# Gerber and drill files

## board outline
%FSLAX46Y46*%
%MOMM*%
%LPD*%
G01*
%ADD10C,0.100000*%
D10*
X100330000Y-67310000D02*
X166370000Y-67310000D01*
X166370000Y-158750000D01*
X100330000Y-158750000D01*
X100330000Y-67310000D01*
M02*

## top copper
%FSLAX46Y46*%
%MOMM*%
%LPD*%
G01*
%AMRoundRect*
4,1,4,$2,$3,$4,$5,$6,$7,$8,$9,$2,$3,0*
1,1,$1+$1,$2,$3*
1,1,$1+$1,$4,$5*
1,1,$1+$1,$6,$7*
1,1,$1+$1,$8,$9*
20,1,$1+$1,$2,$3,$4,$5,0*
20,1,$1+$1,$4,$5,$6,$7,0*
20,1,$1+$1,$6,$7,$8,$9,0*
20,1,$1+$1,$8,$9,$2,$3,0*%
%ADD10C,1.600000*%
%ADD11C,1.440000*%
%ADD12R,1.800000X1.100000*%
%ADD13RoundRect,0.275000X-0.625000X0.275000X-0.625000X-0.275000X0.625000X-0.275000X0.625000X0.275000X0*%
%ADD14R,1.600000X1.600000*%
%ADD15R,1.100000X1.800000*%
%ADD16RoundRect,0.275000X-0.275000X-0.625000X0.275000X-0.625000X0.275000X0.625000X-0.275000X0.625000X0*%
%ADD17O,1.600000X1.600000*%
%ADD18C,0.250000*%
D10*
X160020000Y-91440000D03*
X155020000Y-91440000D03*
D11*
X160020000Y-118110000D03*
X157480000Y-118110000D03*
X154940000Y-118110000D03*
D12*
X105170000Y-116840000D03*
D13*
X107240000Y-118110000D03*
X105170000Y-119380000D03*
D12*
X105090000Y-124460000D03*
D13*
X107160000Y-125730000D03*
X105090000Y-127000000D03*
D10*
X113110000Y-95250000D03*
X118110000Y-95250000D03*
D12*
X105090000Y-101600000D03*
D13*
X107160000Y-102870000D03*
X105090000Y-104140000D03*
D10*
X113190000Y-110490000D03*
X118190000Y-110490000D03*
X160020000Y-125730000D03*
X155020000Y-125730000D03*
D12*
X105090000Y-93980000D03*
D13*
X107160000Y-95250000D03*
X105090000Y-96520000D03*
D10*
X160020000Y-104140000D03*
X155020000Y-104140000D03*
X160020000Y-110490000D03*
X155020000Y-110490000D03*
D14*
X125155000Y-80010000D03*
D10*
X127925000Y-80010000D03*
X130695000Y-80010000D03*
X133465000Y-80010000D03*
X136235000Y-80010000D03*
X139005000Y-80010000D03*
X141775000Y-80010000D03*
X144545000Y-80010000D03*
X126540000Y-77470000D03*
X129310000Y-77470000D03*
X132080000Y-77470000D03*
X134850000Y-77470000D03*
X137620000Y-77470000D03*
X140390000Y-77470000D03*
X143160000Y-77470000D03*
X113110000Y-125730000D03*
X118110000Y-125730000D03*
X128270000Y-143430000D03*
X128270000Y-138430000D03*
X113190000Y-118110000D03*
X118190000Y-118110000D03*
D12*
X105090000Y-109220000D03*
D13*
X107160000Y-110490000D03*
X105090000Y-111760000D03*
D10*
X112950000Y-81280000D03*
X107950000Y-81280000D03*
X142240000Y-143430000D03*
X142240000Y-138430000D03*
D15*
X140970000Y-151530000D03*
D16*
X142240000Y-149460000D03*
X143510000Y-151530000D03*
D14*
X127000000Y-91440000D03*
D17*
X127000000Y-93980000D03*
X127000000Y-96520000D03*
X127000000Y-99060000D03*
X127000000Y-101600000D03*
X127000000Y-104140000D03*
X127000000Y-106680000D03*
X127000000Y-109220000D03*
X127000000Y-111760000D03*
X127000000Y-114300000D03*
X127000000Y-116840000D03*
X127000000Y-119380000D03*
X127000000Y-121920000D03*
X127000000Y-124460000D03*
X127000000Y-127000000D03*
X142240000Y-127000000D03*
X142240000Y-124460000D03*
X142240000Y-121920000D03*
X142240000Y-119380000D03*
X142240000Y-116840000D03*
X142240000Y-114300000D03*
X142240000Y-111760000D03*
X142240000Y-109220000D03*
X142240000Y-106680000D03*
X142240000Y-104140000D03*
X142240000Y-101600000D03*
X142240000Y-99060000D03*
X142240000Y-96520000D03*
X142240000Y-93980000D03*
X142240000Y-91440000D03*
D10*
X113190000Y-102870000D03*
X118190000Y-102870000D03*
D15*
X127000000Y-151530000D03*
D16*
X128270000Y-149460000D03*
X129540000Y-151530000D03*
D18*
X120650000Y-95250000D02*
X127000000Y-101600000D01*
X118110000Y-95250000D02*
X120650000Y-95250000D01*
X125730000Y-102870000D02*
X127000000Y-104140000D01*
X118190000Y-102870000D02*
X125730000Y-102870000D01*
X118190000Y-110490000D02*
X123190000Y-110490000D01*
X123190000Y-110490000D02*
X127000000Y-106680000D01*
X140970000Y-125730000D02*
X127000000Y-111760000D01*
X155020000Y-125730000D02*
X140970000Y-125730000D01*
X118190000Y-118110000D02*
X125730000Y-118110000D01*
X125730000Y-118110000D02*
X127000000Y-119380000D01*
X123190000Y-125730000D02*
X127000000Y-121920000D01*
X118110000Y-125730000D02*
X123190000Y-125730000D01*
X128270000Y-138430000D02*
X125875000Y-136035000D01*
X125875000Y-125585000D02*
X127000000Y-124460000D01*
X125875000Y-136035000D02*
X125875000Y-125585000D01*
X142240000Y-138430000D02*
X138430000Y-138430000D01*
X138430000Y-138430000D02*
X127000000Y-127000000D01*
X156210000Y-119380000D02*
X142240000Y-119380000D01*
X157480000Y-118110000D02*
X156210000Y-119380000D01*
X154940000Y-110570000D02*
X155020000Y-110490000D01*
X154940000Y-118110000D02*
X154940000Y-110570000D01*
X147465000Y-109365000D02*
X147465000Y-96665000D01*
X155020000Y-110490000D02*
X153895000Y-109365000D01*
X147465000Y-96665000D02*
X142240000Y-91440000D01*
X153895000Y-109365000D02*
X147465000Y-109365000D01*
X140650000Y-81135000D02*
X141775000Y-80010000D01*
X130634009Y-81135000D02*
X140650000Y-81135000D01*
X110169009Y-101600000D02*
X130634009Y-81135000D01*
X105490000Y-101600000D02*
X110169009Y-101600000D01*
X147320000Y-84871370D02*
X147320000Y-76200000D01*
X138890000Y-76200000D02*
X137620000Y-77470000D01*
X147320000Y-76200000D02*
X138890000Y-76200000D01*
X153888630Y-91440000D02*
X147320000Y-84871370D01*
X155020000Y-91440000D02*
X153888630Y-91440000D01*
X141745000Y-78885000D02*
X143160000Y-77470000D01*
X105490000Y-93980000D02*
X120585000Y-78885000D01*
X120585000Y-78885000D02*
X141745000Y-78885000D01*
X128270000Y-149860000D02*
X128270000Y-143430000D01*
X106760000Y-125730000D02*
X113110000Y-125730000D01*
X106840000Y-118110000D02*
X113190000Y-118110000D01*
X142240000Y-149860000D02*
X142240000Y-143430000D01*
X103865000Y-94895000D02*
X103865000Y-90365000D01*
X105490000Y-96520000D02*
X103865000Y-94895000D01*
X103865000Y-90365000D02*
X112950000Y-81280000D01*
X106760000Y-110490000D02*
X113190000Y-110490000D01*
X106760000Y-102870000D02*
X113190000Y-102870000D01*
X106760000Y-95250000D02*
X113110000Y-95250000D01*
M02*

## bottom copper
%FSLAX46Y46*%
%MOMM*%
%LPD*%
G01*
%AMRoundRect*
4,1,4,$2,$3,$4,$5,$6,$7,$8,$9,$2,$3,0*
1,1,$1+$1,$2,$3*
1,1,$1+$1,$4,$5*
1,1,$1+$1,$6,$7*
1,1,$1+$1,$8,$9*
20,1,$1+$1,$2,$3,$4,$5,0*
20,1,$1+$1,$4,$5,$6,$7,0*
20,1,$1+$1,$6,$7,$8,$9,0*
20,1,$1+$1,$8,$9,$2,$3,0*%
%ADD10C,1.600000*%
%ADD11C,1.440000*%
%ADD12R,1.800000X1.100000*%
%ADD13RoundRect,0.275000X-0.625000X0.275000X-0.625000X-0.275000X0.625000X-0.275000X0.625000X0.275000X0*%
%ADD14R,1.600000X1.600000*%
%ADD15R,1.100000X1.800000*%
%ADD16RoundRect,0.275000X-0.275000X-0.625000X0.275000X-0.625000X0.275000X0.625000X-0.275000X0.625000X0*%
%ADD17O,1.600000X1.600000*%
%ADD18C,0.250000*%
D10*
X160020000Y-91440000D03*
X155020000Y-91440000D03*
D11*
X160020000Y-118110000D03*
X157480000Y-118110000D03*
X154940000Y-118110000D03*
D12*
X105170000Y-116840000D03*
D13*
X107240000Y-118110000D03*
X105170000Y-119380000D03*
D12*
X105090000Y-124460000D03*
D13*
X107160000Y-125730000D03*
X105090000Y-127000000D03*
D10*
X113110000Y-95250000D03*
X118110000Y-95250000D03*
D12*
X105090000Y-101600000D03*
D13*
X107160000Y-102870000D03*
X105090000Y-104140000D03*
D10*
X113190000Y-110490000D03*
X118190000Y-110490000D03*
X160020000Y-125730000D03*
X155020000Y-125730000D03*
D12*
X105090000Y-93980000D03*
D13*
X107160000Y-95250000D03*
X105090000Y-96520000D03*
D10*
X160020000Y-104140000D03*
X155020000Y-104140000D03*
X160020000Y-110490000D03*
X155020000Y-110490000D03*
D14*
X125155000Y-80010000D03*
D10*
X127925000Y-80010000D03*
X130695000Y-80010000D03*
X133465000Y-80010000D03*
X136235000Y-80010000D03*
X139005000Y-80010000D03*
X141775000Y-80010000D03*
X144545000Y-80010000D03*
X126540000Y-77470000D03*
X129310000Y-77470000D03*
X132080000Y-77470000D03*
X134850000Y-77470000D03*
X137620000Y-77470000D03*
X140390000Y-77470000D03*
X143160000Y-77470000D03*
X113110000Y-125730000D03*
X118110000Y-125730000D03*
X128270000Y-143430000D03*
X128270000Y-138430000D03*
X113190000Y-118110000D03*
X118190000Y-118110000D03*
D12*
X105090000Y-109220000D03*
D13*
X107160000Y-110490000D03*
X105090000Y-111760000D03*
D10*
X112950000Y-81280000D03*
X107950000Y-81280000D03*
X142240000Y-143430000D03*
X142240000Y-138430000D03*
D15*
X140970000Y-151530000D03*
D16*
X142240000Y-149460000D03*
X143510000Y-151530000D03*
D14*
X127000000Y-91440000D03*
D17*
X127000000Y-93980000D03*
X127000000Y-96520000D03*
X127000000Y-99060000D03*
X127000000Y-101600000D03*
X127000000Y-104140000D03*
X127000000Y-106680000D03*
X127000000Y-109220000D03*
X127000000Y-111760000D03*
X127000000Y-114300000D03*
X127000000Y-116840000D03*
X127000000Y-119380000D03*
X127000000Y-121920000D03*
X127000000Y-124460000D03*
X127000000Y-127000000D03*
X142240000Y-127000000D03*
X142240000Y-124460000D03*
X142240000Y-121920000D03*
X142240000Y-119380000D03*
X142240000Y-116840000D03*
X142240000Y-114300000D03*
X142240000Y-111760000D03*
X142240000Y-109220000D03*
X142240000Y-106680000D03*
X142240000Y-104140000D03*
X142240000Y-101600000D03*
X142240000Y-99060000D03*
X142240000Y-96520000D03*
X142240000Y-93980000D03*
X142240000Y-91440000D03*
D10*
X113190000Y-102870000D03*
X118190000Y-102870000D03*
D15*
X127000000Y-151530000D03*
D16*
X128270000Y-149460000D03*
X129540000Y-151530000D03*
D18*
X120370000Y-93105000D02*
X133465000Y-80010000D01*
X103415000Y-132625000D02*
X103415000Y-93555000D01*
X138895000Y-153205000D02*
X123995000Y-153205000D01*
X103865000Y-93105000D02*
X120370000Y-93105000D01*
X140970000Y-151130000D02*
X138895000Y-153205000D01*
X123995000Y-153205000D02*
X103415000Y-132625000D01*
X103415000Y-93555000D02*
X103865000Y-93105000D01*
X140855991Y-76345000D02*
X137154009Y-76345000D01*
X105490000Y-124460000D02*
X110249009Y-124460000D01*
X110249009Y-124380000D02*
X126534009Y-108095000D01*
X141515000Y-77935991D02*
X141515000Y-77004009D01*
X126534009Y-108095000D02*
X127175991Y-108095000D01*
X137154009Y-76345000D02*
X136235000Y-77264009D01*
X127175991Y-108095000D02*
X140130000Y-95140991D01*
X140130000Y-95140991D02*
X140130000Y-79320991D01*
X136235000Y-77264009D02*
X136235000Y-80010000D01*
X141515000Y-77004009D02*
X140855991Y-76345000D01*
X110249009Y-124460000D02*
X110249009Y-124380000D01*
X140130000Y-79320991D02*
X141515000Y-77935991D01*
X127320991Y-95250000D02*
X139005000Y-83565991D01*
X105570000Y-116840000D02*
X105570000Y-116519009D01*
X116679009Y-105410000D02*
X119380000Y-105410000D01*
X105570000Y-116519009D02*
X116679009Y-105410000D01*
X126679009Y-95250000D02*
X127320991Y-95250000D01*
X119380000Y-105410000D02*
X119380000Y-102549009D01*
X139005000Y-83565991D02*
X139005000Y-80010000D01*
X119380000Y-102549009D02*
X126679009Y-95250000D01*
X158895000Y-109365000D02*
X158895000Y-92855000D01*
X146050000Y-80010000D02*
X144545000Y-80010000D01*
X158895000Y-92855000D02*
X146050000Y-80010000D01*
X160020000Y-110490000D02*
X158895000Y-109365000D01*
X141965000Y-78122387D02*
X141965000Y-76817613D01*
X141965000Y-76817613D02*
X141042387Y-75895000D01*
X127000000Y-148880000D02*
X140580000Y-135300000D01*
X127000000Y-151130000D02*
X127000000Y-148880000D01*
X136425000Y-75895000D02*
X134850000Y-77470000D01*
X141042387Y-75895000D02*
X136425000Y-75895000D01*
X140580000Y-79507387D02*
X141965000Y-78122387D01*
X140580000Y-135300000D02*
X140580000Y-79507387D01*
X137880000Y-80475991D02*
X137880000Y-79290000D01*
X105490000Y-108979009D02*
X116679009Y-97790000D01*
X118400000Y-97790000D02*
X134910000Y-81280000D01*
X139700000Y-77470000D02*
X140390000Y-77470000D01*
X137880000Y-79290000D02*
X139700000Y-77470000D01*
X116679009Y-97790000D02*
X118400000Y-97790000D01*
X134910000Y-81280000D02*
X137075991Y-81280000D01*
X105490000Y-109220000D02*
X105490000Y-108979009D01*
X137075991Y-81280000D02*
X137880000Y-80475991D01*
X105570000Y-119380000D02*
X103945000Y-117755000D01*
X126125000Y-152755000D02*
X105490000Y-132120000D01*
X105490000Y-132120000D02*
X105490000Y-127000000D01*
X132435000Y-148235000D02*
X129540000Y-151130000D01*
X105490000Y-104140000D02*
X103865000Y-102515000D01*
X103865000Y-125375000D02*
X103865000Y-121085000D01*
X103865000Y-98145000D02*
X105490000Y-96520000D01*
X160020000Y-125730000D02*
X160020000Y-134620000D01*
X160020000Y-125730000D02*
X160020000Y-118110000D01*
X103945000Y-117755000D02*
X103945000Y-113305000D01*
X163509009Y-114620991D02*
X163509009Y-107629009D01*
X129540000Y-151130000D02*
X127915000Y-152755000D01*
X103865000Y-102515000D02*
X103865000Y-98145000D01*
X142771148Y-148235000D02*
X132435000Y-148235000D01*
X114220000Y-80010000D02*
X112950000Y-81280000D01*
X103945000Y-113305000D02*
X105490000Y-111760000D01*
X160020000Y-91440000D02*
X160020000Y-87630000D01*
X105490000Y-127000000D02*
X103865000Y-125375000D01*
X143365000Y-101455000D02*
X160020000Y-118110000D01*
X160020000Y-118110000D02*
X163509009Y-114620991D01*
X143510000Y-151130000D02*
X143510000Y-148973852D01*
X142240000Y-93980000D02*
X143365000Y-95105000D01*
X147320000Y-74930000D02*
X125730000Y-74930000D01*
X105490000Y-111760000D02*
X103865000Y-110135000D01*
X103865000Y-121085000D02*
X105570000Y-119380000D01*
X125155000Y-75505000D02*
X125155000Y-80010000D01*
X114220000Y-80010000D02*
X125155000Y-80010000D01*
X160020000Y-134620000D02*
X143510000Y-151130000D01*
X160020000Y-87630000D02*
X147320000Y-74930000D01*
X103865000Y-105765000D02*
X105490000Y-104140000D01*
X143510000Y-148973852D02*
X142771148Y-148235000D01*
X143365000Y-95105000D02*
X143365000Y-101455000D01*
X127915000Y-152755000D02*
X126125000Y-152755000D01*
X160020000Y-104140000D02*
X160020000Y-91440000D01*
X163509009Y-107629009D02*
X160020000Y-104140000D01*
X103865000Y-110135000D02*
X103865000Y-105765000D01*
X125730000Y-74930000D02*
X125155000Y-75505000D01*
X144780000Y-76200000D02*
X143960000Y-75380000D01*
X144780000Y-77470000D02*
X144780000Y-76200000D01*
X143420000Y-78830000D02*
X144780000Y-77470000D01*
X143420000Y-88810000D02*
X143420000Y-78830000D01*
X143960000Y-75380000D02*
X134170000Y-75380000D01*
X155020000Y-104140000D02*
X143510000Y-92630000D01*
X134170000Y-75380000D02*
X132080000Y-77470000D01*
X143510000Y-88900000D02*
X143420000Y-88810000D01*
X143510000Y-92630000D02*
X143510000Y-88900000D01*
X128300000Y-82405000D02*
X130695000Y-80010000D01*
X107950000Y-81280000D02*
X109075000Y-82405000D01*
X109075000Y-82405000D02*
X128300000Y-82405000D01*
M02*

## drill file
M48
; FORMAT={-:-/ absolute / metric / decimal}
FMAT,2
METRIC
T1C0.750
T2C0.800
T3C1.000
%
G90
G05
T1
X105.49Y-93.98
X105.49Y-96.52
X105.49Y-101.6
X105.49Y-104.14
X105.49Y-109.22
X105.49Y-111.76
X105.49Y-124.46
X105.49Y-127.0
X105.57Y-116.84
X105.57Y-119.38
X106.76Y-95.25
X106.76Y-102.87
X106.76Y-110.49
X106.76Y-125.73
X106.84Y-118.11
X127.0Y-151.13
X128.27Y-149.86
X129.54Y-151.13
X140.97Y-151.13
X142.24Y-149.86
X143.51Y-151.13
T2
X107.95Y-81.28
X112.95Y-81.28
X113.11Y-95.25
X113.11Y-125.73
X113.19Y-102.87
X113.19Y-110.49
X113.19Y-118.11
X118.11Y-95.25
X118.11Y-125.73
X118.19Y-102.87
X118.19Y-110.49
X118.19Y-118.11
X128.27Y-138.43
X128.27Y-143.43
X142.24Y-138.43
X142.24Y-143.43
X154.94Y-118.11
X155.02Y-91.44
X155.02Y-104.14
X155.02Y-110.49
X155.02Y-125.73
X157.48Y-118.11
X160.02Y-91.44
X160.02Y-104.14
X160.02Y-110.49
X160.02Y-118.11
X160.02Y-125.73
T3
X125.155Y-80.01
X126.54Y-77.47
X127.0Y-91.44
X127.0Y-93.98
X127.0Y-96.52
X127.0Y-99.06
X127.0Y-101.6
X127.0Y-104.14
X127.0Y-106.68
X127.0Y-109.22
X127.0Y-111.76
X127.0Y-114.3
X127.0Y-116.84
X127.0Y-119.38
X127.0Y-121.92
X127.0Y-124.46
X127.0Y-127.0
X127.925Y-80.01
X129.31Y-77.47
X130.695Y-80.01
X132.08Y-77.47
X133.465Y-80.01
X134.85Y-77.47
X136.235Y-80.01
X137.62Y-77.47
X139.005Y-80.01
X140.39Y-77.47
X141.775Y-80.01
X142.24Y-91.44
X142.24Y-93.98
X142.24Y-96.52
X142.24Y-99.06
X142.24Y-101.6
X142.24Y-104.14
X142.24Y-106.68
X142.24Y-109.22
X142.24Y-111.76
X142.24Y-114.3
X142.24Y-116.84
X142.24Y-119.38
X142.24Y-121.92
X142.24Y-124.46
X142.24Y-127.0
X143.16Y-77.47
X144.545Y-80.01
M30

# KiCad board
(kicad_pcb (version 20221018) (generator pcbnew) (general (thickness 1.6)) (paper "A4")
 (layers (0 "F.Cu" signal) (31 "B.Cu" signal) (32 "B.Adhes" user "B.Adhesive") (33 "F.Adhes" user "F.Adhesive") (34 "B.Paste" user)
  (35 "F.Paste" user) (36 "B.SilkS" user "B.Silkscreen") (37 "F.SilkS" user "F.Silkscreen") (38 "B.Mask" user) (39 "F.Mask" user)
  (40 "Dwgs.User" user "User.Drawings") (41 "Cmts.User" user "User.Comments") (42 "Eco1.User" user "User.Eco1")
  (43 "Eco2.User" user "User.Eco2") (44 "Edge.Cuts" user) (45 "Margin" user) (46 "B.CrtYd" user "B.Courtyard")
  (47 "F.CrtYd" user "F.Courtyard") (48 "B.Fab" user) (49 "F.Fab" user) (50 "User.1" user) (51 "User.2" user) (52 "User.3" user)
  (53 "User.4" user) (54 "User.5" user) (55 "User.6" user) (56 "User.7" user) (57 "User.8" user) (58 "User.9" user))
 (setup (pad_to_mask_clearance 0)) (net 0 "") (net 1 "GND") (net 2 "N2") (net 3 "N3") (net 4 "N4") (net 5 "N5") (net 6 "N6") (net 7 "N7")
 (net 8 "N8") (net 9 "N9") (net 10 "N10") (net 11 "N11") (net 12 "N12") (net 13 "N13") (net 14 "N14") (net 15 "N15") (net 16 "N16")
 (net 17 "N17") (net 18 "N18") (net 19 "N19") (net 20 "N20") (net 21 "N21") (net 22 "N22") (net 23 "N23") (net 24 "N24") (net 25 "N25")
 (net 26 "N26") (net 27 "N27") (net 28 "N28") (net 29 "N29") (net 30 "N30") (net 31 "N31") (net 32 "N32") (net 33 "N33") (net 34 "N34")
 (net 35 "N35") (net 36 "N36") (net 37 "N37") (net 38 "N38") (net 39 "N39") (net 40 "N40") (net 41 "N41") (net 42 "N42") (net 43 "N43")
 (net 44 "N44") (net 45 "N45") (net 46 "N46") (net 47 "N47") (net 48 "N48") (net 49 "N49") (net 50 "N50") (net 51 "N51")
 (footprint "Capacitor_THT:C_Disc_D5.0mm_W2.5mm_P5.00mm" (layer "F.Cu") (at 160.02 91.44 180)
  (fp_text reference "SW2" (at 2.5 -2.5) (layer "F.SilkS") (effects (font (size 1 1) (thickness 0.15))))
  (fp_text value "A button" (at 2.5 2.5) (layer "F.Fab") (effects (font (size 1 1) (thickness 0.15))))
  (pad "1" thru_hole circle (at 0 0 180) (size 1.6 1.6) (drill 0.8) (layers "*.Cu" "*.Mask") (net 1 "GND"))
  (pad "2" thru_hole circle (at 5 0 180) (size 1.6 1.6) (drill 0.8) (layers "*.Cu" "*.Mask") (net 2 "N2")))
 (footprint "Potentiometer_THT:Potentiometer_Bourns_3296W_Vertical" (layer "F.Cu") (at 160.02 118.11)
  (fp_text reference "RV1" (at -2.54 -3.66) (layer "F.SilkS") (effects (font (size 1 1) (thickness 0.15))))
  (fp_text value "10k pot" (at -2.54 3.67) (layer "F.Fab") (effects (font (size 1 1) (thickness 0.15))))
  (pad "1" thru_hole circle (at 0 0) (size 1.44 1.44) (drill 0.8) (layers "*.Cu" "*.Mask") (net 1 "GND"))
  (pad "2" thru_hole circle (at -2.54 0) (size 1.44 1.44) (drill 0.8) (layers "*.Cu" "*.Mask") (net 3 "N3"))
  (pad "3" thru_hole circle (at -5.08 0) (size 1.44 1.44) (drill 0.8) (layers "*.Cu" "*.Mask") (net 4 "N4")))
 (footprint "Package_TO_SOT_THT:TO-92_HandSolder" (layer "F.Cu") (at 105.57 116.84 -90)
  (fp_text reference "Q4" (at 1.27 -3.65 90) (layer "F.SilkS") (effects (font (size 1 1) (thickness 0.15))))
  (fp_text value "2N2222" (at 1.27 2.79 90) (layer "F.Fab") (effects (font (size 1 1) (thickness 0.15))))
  (pad "1" thru_hole rect (at 0 0 270) (size 1.1 1.8) (drill 0.75 (offset 0 0.4)) (layers "*.Cu" "*.Mask") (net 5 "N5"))
  (pad "2" thru_hole roundrect (at 1.27 -1.27 270) (size 1.1 1.8) (drill 0.75 (offset 0 -0.4)) (layers "*.Cu" "*.Mask")
   (roundrect_rratio 0.25) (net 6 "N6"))
  (pad "3" thru_hole roundrect (at 2.54 0 270) (size 1.1 1.8) (drill 0.75 (offset 0 0.4)) (layers "*.Cu" "*.Mask") (roundrect_rratio 0.25)
   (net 1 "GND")))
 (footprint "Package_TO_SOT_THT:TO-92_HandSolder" (layer "F.Cu") (at 105.49 124.46 -90)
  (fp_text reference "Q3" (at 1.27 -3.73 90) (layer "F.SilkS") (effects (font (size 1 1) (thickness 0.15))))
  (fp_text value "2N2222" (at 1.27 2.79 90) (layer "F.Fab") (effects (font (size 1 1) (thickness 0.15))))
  (pad "1" thru_hole rect (at 0 0 270) (size 1.1 1.8) (drill 0.75 (offset 0 0.4)) (layers "*.Cu" "*.Mask") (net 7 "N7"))
  (pad "2" thru_hole roundrect (at 1.27 -1.27 270) (size 1.1 1.8) (drill 0.75 (offset 0 -0.4)) (layers "*.Cu" "*.Mask")
   (roundrect_rratio 0.25) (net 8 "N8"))
  (pad "3" thru_hole roundrect (at 2.54 0 270) (size 1.1 1.8) (drill 0.75 (offset 0 0.4)) (layers "*.Cu" "*.Mask") (roundrect_rratio 0.25)
   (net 1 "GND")))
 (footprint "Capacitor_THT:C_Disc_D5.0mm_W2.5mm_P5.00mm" (layer "F.Cu") (at 113.11 95.25)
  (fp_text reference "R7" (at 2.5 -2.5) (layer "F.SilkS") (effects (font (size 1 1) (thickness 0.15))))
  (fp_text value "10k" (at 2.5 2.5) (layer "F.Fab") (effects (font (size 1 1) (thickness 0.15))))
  (pad "1" thru_hole circle (at 0 0) (size 1.6 1.6) (drill 0.8) (layers "*.Cu" "*.Mask") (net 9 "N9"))
  (pad "2" thru_hole circle (at 5 0) (size 1.6 1.6) (drill 0.8) (layers "*.Cu" "*.Mask") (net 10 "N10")))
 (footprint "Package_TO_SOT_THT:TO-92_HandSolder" (layer "F.Cu") (at 105.49 101.6 -90)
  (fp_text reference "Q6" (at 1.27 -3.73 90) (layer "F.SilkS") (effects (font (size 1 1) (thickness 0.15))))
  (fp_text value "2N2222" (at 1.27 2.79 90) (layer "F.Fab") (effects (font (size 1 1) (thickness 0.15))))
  (pad "1" thru_hole rect (at 0 0 270) (size 1.1 1.8) (drill 0.75 (offset 0 0.4)) (layers "*.Cu" "*.Mask") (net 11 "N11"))
  (pad "2" thru_hole roundrect (at 1.27 -1.27 270) (size 1.1 1.8) (drill 0.75 (offset 0 -0.4)) (layers "*.Cu" "*.Mask")
   (roundrect_rratio 0.25) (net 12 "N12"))
  (pad "3" thru_hole roundrect (at 2.54 0 270) (size 1.1 1.8) (drill 0.75 (offset 0 0.4)) (layers "*.Cu" "*.Mask") (roundrect_rratio 0.25)
   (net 1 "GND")))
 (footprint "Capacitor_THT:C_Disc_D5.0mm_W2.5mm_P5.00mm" (layer "F.Cu") (at 113.19 110.49)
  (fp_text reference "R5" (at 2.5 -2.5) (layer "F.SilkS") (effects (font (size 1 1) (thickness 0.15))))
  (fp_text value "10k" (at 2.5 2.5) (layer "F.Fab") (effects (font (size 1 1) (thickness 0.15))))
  (pad "1" thru_hole circle (at 0 0) (size 1.6 1.6) (drill 0.8) (layers "*.Cu" "*.Mask") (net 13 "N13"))
  (pad "2" thru_hole circle (at 5 0) (size 1.6 1.6) (drill 0.8) (layers "*.Cu" "*.Mask") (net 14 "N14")))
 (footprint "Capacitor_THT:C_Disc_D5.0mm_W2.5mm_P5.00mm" (layer "F.Cu") (at 160.02 125.73 180)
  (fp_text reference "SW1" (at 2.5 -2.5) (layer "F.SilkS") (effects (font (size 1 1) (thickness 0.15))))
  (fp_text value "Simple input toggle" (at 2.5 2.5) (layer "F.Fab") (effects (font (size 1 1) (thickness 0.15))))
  (pad "1" thru_hole circle (at 0 0 180) (size 1.6 1.6) (drill 0.8) (layers "*.Cu" "*.Mask") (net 1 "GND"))
  (pad "2" thru_hole circle (at 5 0 180) (size 1.6 1.6) (drill 0.8) (layers "*.Cu" "*.Mask") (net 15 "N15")))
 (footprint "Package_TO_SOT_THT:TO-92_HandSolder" (layer "F.Cu") (at 105.49 93.98 -90)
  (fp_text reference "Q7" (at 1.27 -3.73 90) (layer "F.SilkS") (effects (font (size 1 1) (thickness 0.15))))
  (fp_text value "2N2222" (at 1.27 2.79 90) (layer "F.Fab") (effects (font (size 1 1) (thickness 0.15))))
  (pad "1" thru_hole rect (at 0 0 270) (size 1.1 1.8) (drill 0.75 (offset 0 0.4)) (layers "*.Cu" "*.Mask") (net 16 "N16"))
  (pad "2" thru_hole roundrect (at 1.27 -1.27 270) (size 1.1 1.8) (drill 0.75 (offset 0 -0.4)) (layers "*.Cu" "*.Mask")
   (roundrect_rratio 0.25) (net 9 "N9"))
  (pad "3" thru_hole roundrect (at 2.54 0 270) (size 1.1 1.8) (drill 0.75 (offset 0 0.4)) (layers "*.Cu" "*.Mask") (roundrect_rratio 0.25)
   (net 1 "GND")))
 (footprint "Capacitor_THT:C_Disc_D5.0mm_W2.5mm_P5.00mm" (layer "F.Cu") (at 160.02 104.14 180)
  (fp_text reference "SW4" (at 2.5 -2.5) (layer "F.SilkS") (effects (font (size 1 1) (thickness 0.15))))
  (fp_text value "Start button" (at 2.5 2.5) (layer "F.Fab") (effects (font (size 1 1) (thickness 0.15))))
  (pad "1" thru_hole circle (at 0 0 180) (size 1.6 1.6) (drill 0.8) (layers "*.Cu" "*.Mask") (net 1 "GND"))
  (pad "2" thru_hole circle (at 5 0 180) (size 1.6 1.6) (drill 0.8) (layers "*.Cu" "*.Mask") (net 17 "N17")))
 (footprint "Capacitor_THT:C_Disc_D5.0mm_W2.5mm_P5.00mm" (layer "F.Cu") (at 160.02 110.49 180)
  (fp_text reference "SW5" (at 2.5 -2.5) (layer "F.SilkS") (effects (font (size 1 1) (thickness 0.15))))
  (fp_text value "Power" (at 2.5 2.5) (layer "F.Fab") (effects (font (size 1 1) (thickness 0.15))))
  (pad "1" thru_hole circle (at 0 0 180) (size 1.6 1.6) (drill 0.8) (layers "*.Cu" "*.Mask") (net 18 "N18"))
  (pad "2" thru_hole circle (at 5 0 180) (size 1.6 1.6) (drill 0.8) (layers "*.Cu" "*.Mask") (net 4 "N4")))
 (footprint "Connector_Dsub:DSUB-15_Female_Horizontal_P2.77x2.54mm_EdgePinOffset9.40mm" (layer "F.Cu") (at 125.155 80.01 180)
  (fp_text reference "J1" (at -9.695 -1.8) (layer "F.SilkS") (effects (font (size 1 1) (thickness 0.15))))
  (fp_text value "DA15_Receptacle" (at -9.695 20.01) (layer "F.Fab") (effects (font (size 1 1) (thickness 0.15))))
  (pad "1" thru_hole rect (at 0 0 180) (size 1.6 1.6) (drill 1) (layers "*.Cu" "*.Mask") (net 1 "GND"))
  (pad "2" thru_hole circle (at -2.77 0 180) (size 1.6 1.6) (drill 1) (layers "*.Cu" "*.Mask") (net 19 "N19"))
  (pad "3" thru_hole circle (at -5.54 0 180) (size 1.6 1.6) (drill 1) (layers "*.Cu" "*.Mask") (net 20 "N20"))
  (pad "4" thru_hole circle (at -8.31 0 180) (size 1.6 1.6) (drill 1) (layers "*.Cu" "*.Mask") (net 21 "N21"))
  (pad "5" thru_hole circle (at -11.08 0 180) (size 1.6 1.6) (drill 1) (layers "*.Cu" "*.Mask") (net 7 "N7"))
  (pad "6" thru_hole circle (at -13.85 0 180) (size 1.6 1.6) (drill 1) (layers "*.Cu" "*.Mask") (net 5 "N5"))
  (pad "7" thru_hole circle (at -16.62 0 180) (size 1.6 1.6) (drill 1) (layers "*.Cu" "*.Mask") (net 11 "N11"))
  (pad "8" thru_hole circle (at -19.39 0 180) (size 1.6 1.6) (drill 1) (layers "*.Cu" "*.Mask") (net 18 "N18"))
  (pad "9" thru_hole circle (at -1.385 2.54 180) (size 1.6 1.6) (drill 1) (layers "*.Cu" "*.Mask") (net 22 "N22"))
  (pad "10" thru_hole circle (at -4.155 2.54 180) (size 1.6 1.6) (drill 1) (layers "*.Cu" "*.Mask") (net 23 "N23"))
  (pad "11" thru_hole circle (at -6.925 2.54 180) (size 1.6 1.6) (drill 1) (layers "*.Cu" "*.Mask") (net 17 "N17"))
  (pad "12" thru_hole circle (at -9.695 2.54 180) (size 1.6 1.6) (drill 1) (layers "*.Cu" "*.Mask") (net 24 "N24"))
  (pad "13" thru_hole circle (at -12.465 2.54 180) (size 1.6 1.6) (drill 1) (layers "*.Cu" "*.Mask") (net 2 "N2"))
  (pad "14" thru_hole circle (at -15.235 2.54 180) (size 1.6 1.6) (drill 1) (layers "*.Cu" "*.Mask") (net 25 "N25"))
  (pad "15" thru_hole circle (at -18.005 2.54 180) (size 1.6 1.6) (drill 1) (layers "*.Cu" "*.Mask") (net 16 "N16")))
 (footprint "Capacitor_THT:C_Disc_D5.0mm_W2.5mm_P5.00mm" (layer "F.Cu") (at 113.11 125.73)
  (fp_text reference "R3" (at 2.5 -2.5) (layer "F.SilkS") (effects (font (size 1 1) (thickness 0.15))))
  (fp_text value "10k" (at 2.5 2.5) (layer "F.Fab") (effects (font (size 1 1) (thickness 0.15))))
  (pad "1" thru_hole circle (at 0 0) (size 1.6 1.6) (drill 0.8) (layers "*.Cu" "*.Mask") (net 8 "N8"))
  (pad "2" thru_hole circle (at 5 0) (size 1.6 1.6) (drill 0.8) (layers "*.Cu" "*.Mask") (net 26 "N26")))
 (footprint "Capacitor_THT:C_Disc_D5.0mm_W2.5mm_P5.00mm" (layer "F.Cu") (at 128.27 143.43 90)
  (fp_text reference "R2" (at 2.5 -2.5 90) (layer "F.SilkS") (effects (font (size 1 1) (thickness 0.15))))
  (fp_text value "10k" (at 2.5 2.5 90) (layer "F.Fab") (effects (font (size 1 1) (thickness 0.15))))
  (pad "1" thru_hole circle (at 0 0 90) (size 1.6 1.6) (drill 0.8) (layers "*.Cu" "*.Mask") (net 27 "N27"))
  (pad "2" thru_hole circle (at 5 0 90) (size 1.6 1.6) (drill 0.8) (layers "*.Cu" "*.Mask") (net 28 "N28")))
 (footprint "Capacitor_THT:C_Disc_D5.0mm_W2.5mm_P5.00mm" (layer "F.Cu") (at 113.19 118.11)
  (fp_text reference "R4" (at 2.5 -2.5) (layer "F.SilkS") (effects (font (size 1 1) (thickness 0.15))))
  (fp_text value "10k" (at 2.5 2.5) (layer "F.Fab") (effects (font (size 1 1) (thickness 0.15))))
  (pad "1" thru_hole circle (at 0 0) (size 1.6 1.6) (drill 0.8) (layers "*.Cu" "*.Mask") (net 6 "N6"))
  (pad "2" thru_hole circle (at 5 0) (size 1.6 1.6) (drill 0.8) (layers "*.Cu" "*.Mask") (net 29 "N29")))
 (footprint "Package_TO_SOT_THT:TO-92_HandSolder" (layer "F.Cu") (at 105.49 109.22 -90)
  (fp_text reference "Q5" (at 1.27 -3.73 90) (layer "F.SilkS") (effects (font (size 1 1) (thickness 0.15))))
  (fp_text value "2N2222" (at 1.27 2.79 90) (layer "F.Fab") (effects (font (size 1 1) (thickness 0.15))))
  (pad "1" thru_hole rect (at 0 0 270) (size 1.1 1.8) (drill 0.75 (offset 0 0.4)) (layers "*.Cu" "*.Mask") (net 25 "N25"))
  (pad "2" thru_hole roundrect (at 1.27 -1.27 270) (size 1.1 1.8) (drill 0.75 (offset 0 -0.4)) (layers "*.Cu" "*.Mask")
   (roundrect_rratio 0.25) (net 13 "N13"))
  (pad "3" thru_hole roundrect (at 2.54 0 270) (size 1.1 1.8) (drill 0.75 (offset 0 0.4)) (layers "*.Cu" "*.Mask") (roundrect_rratio 0.25)
   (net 1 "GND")))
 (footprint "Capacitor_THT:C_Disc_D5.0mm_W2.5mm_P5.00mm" (layer "F.Cu") (at 112.95 81.28 180)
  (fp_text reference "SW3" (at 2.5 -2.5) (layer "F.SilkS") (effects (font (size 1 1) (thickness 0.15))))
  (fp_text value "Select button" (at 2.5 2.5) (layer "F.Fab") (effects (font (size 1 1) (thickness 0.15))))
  (pad "1" thru_hole circle (at 0 0 180) (size 1.6 1.6) (drill 0.8) (layers "*.Cu" "*.Mask") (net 1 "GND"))
  (pad "2" thru_hole circle (at 5 0 180) (size 1.6 1.6) (drill 0.8) (layers "*.Cu" "*.Mask") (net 20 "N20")))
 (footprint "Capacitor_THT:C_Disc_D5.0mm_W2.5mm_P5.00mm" (layer "F.Cu") (at 142.24 143.43 90)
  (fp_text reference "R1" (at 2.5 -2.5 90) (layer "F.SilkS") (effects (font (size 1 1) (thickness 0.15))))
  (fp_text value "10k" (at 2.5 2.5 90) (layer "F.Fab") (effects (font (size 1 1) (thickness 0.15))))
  (pad "1" thru_hole circle (at 0 0 90) (size 1.6 1.6) (drill 0.8) (layers "*.Cu" "*.Mask") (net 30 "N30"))
  (pad "2" thru_hole circle (at 5 0 90) (size 1.6 1.6) (drill 0.8) (layers "*.Cu" "*.Mask") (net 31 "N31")))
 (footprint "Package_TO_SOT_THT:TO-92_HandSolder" (layer "F.Cu") (at 140.97 151.13)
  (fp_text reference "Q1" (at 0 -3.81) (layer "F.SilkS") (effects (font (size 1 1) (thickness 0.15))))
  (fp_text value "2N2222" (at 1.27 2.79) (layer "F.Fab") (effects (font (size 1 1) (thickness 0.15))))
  (pad "1" thru_hole rect (at 0 0) (size 1.1 1.8) (drill 0.75 (offset 0 0.4)) (layers "*.Cu" "*.Mask") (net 21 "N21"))
  (pad "2" thru_hole roundrect (at 1.27 -1.27) (size 1.1 1.8) (drill 0.75 (offset 0 -0.4)) (layers "*.Cu" "*.Mask") (roundrect_rratio 0.25)
   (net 30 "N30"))
  (pad "3" thru_hole roundrect (at 2.54 0) (size 1.1 1.8) (drill 0.75 (offset 0 0.4)) (layers "*.Cu" "*.Mask") (roundrect_rratio 0.25)
   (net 1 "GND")))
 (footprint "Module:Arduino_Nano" (layer "F.Cu") (at 127 91.44)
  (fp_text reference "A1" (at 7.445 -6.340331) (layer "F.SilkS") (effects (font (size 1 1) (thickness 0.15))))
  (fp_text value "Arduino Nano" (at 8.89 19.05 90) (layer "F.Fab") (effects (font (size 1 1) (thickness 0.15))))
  (pad "1" thru_hole rect (at 0 0) (size 1.6 1.6) (drill 1) (layers "*.Cu" "*.Mask") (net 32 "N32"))
  (pad "2" thru_hole oval (at 0 2.54) (size 1.6 1.6) (drill 1) (layers "*.Cu" "*.Mask") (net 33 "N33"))
  (pad "3" thru_hole oval (at 0 5.08) (size 1.6 1.6) (drill 1) (layers "*.Cu" "*.Mask") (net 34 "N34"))
  (pad "4" thru_hole oval (at 0 7.62) (size 1.6 1.6) (drill 1) (layers "*.Cu" "*.Mask") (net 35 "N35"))
  (pad "5" thru_hole oval (at 0 10.16) (size 1.6 1.6) (drill 1) (layers "*.Cu" "*.Mask") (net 10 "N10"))
  (pad "6" thru_hole oval (at 0 12.7) (size 1.6 1.6) (drill 1) (layers "*.Cu" "*.Mask") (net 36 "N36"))
  (pad "7" thru_hole oval (at 0 15.24) (size 1.6 1.6) (drill 1) (layers "*.Cu" "*.Mask") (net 14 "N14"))
  (pad "8" thru_hole oval (at 0 17.78) (size 1.6 1.6) (drill 1) (layers "*.Cu" "*.Mask") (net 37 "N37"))
  (pad "9" thru_hole oval (at 0 20.32) (size 1.6 1.6) (drill 1) (layers "*.Cu" "*.Mask") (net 15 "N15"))
  (pad "10" thru_hole oval (at 0 22.86) (size 1.6 1.6) (drill 1) (layers "*.Cu" "*.Mask") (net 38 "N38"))
  (pad "11" thru_hole oval (at 0 25.4) (size 1.6 1.6) (drill 1) (layers "*.Cu" "*.Mask") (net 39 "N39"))
  (pad "12" thru_hole oval (at 0 27.94) (size 1.6 1.6) (drill 1) (layers "*.Cu" "*.Mask") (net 29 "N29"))
  (pad "13" thru_hole oval (at 0 30.48) (size 1.6 1.6) (drill 1) (layers "*.Cu" "*.Mask") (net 26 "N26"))
  (pad "14" thru_hole oval (at 0 33.02) (size 1.6 1.6) (drill 1) (layers "*.Cu" "*.Mask") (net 28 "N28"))
  (pad "15" thru_hole oval (at 0 35.56) (size 1.6 1.6) (drill 1) (layers "*.Cu" "*.Mask") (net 31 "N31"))
  (pad "16" thru_hole oval (at 15.24 35.56) (size 1.6 1.6) (drill 1) (layers "*.Cu" "*.Mask") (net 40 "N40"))
  (pad "17" thru_hole oval (at 15.24 33.02) (size 1.6 1.6) (drill 1) (layers "*.Cu" "*.Mask") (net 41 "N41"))
  (pad "18" thru_hole oval (at 15.24 30.48) (size 1.6 1.6) (drill 1) (layers "*.Cu" "*.Mask") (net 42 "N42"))
  (pad "19" thru_hole oval (at 15.24 27.94) (size 1.6 1.6) (drill 1) (layers "*.Cu" "*.Mask") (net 3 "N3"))
  (pad "20" thru_hole oval (at 15.24 25.4) (size 1.6 1.6) (drill 1) (layers "*.Cu" "*.Mask") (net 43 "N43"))
  (pad "21" thru_hole oval (at 15.24 22.86) (size 1.6 1.6) (drill 1) (layers "*.Cu" "*.Mask") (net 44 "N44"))
  (pad "22" thru_hole oval (at 15.24 20.32) (size 1.6 1.6) (drill 1) (layers "*.Cu" "*.Mask") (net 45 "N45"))
  (pad "23" thru_hole oval (at 15.24 17.78) (size 1.6 1.6) (drill 1) (layers "*.Cu" "*.Mask") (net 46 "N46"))
  (pad "24" thru_hole oval (at 15.24 15.24) (size 1.6 1.6) (drill 1) (layers "*.Cu" "*.Mask") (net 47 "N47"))
  (pad "25" thru_hole oval (at 15.24 12.7) (size 1.6 1.6) (drill 1) (layers "*.Cu" "*.Mask") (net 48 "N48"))
  (pad "26" thru_hole oval (at 15.24 10.16) (size 1.6 1.6) (drill 1) (layers "*.Cu" "*.Mask") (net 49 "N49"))
  (pad "27" thru_hole oval (at 15.24 7.62) (size 1.6 1.6) (drill 1) (layers "*.Cu" "*.Mask") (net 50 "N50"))
  (pad "28" thru_hole oval (at 15.24 5.08) (size 1.6 1.6) (drill 1) (layers "*.Cu" "*.Mask") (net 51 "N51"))
  (pad "29" thru_hole oval (at 15.24 2.54) (size 1.6 1.6) (drill 1) (layers "*.Cu" "*.Mask") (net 1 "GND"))
  (pad "30" thru_hole oval (at 15.24 0) (size 1.6 1.6) (drill 1) (layers "*.Cu" "*.Mask") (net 4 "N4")))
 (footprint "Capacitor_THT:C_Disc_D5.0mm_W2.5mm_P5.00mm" (layer "F.Cu") (at 113.19 102.87)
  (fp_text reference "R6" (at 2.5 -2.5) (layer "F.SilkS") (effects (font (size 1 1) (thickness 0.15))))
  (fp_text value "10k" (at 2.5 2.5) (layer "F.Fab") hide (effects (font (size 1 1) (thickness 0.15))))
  (pad "1" thru_hole circle (at 0 0) (size 1.6 1.6) (drill 0.8) (layers "*.Cu" "*.Mask") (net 12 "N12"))
  (pad "2" thru_hole circle (at 5 0) (size 1.6 1.6) (drill 0.8) (layers "*.Cu" "*.Mask") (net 36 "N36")))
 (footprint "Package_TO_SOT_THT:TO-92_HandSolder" (layer "F.Cu") (at 127 151.13)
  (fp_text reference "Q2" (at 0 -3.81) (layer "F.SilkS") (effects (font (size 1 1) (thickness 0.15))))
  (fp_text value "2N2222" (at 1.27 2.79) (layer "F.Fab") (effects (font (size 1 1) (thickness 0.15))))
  (pad "1" thru_hole rect (at 0 0) (size 1.1 1.8) (drill 0.75 (offset 0 0.4)) (layers "*.Cu" "*.Mask") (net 24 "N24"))
  (pad "2" thru_hole roundrect (at 1.27 -1.27) (size 1.1 1.8) (drill 0.75 (offset 0 -0.4)) (layers "*.Cu" "*.Mask") (roundrect_rratio 0.25)
   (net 27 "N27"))
  (pad "3" thru_hole roundrect (at 2.54 0) (size 1.1 1.8) (drill 0.75 (offset 0 0.4)) (layers "*.Cu" "*.Mask") (roundrect_rratio 0.25)
   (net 1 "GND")))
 (gr_rect (start 100.33 67.31) (end 166.37 158.75) (stroke (width 0.1) (type default)) (fill none) (layer "Edge.Cuts"))
 (segment (start 120.65 95.25) (end 127 101.6) (width 0.25) (layer "F.Cu") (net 10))
 (segment (start 118.11 95.25) (end 120.65 95.25) (width 0.25) (layer "F.Cu") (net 10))
 (segment (start 125.73 102.87) (end 127 104.14) (width 0.25) (layer "F.Cu") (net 36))
 (segment (start 118.19 102.87) (end 125.73 102.87) (width 0.25) (layer "F.Cu") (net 36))
 (segment (start 118.19 110.49) (end 123.19 110.49) (width 0.25) (layer "F.Cu") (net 14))
 (segment (start 123.19 110.49) (end 127 106.68) (width 0.25) (layer "F.Cu") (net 14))
 (segment (start 140.97 125.73) (end 127 111.76) (width 0.25) (layer "F.Cu") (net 15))
 (segment (start 155.02 125.73) (end 140.97 125.73) (width 0.25) (layer "F.Cu") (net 15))
 (segment (start 118.19 118.11) (end 125.73 118.11) (width 0.25) (layer "F.Cu") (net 29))
 (segment (start 125.73 118.11) (end 127 119.38) (width 0.25) (layer "F.Cu") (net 29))
 (segment (start 123.19 125.73) (end 127 121.92) (width 0.25) (layer "F.Cu") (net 26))
 (segment (start 118.11 125.73) (end 123.19 125.73) (width 0.25) (layer "F.Cu") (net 26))
 (segment (start 128.27 138.43) (end 125.875 136.035) (width 0.25) (layer "F.Cu") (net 28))
 (segment (start 125.875 125.585) (end 127 124.46) (width 0.25) (layer "F.Cu") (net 28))
 (segment (start 125.875 136.035) (end 125.875 125.585) (width 0.25) (layer "F.Cu") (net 28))
 (segment (start 142.24 138.43) (end 138.43 138.43) (width 0.25) (layer "F.Cu") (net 31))
 (segment (start 138.43 138.43) (end 127 127) (width 0.25) (layer "F.Cu") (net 31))
 (segment (start 156.21 119.38) (end 142.24 119.38) (width 0.25) (layer "F.Cu") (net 3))
 (segment (start 157.48 118.11) (end 156.21 119.38) (width 0.25) (layer "F.Cu") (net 3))
 (segment (start 154.94 110.57) (end 155.02 110.49) (width 0.25) (layer "F.Cu") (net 4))
 (segment (start 154.94 118.11) (end 154.94 110.57) (width 0.25) (layer "F.Cu") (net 4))
 (segment (start 147.465 109.365) (end 147.465 96.665) (width 0.25) (layer "F.Cu") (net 4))
 (segment (start 155.02 110.49) (end 153.895 109.365) (width 0.25) (layer "F.Cu") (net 4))
 (segment (start 147.465 96.665) (end 142.24 91.44) (width 0.25) (layer "F.Cu") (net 4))
 (segment (start 153.895 109.365) (end 147.465 109.365) (width 0.25) (layer "F.Cu") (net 4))
 (segment (start 120.37 93.105) (end 133.465 80.01) (width 0.25) (layer "B.Cu") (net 21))
 (segment (start 103.415 132.625) (end 103.415 93.555) (width 0.25) (layer "B.Cu") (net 21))
 (segment (start 138.895 153.205) (end 123.995 153.205) (width 0.25) (layer "B.Cu") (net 21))
 (segment (start 103.865 93.105) (end 120.37 93.105) (width 0.25) (layer "B.Cu") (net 21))
 (segment (start 140.97 151.13) (end 138.895 153.205) (width 0.25) (layer "B.Cu") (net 21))
 (segment (start 123.995 153.205) (end 103.415 132.625) (width 0.25) (layer "B.Cu") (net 21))
 (segment (start 103.415 93.555) (end 103.865 93.105) (width 0.25) (layer "B.Cu") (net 21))
 (segment (start 140.855991 76.345) (end 137.154009 76.345) (width 0.25) (layer "B.Cu") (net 7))
 (segment (start 105.49 124.46) (end 110.249009 124.46) (width 0.25) (layer "B.Cu") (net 7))
 (segment (start 110.249009 124.38) (end 126.534009 108.095) (width 0.25) (layer "B.Cu") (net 7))
 (segment (start 141.515 77.935991) (end 141.515 77.004009) (width 0.25) (layer "B.Cu") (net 7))
 (segment (start 126.534009 108.095) (end 127.175991 108.095) (width 0.25) (layer "B.Cu") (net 7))
 (segment (start 137.154009 76.345) (end 136.235 77.264009) (width 0.25) (layer "B.Cu") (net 7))
 (segment (start 127.175991 108.095) (end 140.13 95.140991) (width 0.25) (layer "B.Cu") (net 7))
 (segment (start 140.13 95.140991) (end 140.13 79.320991) (width 0.25) (layer "B.Cu") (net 7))
 (segment (start 136.235 77.264009) (end 136.235 80.01) (width 0.25) (layer "B.Cu") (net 7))
 (segment (start 141.515 77.004009) (end 140.855991 76.345) (width 0.25) (layer "B.Cu") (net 7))
 (segment (start 110.249009 124.46) (end 110.249009 124.38) (width 0.25) (layer "B.Cu") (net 7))
 (segment (start 140.13 79.320991) (end 141.515 77.935991) (width 0.25) (layer "B.Cu") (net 7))
 (segment (start 127.320991 95.25) (end 139.005 83.565991) (width 0.25) (layer "B.Cu") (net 5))
 (segment (start 105.57 116.84) (end 105.57 116.519009) (width 0.25) (layer "B.Cu") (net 5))
 (segment (start 116.679009 105.41) (end 119.38 105.41) (width 0.25) (layer "B.Cu") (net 5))
 (segment (start 105.57 116.519009) (end 116.679009 105.41) (width 0.25) (layer "B.Cu") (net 5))
 (segment (start 126.679009 95.25) (end 127.320991 95.25) (width 0.25) (layer "B.Cu") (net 5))
 (segment (start 119.38 105.41) (end 119.38 102.549009) (width 0.25) (layer "B.Cu") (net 5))
 (segment (start 139.005 83.565991) (end 139.005 80.01) (width 0.25) (layer "B.Cu") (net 5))
 (segment (start 119.38 102.549009) (end 126.679009 95.25) (width 0.25) (layer "B.Cu") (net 5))
 (segment (start 140.65 81.135) (end 141.775 80.01) (width 0.25) (layer "F.Cu") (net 11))
 (segment (start 130.634009 81.135) (end 140.65 81.135) (width 0.25) (layer "F.Cu") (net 11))
 (segment (start 110.169009 101.6) (end 130.634009 81.135) (width 0.25) (layer "F.Cu") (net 11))
 (segment (start 105.49 101.6) (end 110.169009 101.6) (width 0.25) (layer "F.Cu") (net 11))
 (segment (start 158.895 109.365) (end 158.895 92.855) (width 0.25) (layer "B.Cu") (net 18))
 (segment (start 146.05 80.01) (end 144.545 80.01) (width 0.25) (layer "B.Cu") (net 18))
 (segment (start 158.895 92.855) (end 146.05 80.01) (width 0.25) (layer "B.Cu") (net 18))
 (segment (start 160.02 110.49) (end 158.895 109.365) (width 0.25) (layer "B.Cu") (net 18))
 (segment (start 141.965 78.122387) (end 141.965 76.817613) (width 0.25) (layer "B.Cu") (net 24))
 (segment (start 141.965 76.817613) (end 141.042387 75.895) (width 0.25) (layer "B.Cu") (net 24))
 (segment (start 127 148.88) (end 140.58 135.3) (width 0.25) (layer "B.Cu") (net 24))
 (segment (start 127 151.13) (end 127 148.88) (width 0.25) (layer "B.Cu") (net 24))
 (segment (start 136.425 75.895) (end 134.85 77.47) (width 0.25) (layer "B.Cu") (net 24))
 (segment (start 141.042387 75.895) (end 136.425 75.895) (width 0.25) (layer "B.Cu") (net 24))
 (segment (start 140.58 79.507387) (end 141.965 78.122387) (width 0.25) (layer "B.Cu") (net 24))
 (segment (start 140.58 135.3) (end 140.58 79.507387) (width 0.25) (layer "B.Cu") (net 24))
 (segment (start 147.32 84.87137) (end 147.32 76.2) (width 0.25) (layer "F.Cu") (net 2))
 (segment (start 138.89 76.2) (end 137.62 77.47) (width 0.25) (layer "F.Cu") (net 2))
 (segment (start 147.32 76.2) (end 138.89 76.2) (width 0.25) (layer "F.Cu") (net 2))
 (segment (start 153.88863 91.44) (end 147.32 84.87137) (width 0.25) (layer "F.Cu") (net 2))
 (segment (start 155.02 91.44) (end 153.88863 91.44) (width 0.25) (layer "F.Cu") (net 2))
 (segment (start 137.88 80.475991) (end 137.88 79.29) (width 0.25) (layer "B.Cu") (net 25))
 (segment (start 105.49 108.979009) (end 116.679009 97.79) (width 0.25) (layer "B.Cu") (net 25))
 (segment (start 118.4 97.79) (end 134.91 81.28) (width 0.25) (layer "B.Cu") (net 25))
 (segment (start 139.7 77.47) (end 140.39 77.47) (width 0.25) (layer "B.Cu") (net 25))
 (segment (start 137.88 79.29) (end 139.7 77.47) (width 0.25) (layer "B.Cu") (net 25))
 (segment (start 116.679009 97.79) (end 118.4 97.79) (width 0.25) (layer "B.Cu") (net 25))
 (segment (start 134.91 81.28) (end 137.075991 81.28) (width 0.25) (layer "B.Cu") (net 25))
 (segment (start 105.49 109.22) (end 105.49 108.979009) (width 0.25) (layer "B.Cu") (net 25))
 (segment (start 137.075991 81.28) (end 137.88 80.475991) (width 0.25) (layer "B.Cu") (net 25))
 (segment (start 141.745 78.885) (end 143.16 77.47) (width 0.25) (layer "F.Cu") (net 16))
 (segment (start 105.49 93.98) (end 120.585 78.885) (width 0.25) (layer "F.Cu") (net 16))
 (segment (start 120.585 78.885) (end 141.745 78.885) (width 0.25) (layer "F.Cu") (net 16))
 (segment (start 128.27 149.86) (end 128.27 143.43) (width 0.25) (layer "F.Cu") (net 27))
 (segment (start 106.76 125.73) (end 113.11 125.73) (width 0.25) (layer "F.Cu") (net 8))
 (segment (start 106.84 118.11) (end 113.19 118.11) (width 0.25) (layer "F.Cu") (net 6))
 (segment (start 142.24 149.86) (end 142.24 143.43) (width 0.25) (layer "F.Cu") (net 30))
 (segment (start 103.865 94.895) (end 103.865 90.365) (width 0.25) (layer "F.Cu") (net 1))
 (segment (start 105.49 96.52) (end 103.865 94.895) (width 0.25) (layer "F.Cu") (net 1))
 (segment (start 103.865 90.365) (end 112.95 81.28) (width 0.25) (layer "F.Cu") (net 1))
 (segment (start 105.57 119.38) (end 103.945 117.755) (width 0.25) (layer "B.Cu") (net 1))
 (segment (start 126.125 152.755) (end 105.49 132.12) (width 0.25) (layer "B.Cu") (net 1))
 (segment (start 105.49 132.12) (end 105.49 127) (width 0.25) (layer "B.Cu") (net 1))
 (segment (start 132.435 148.235) (end 129.54 151.13) (width 0.25) (layer "B.Cu") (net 1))
 (segment (start 105.49 104.14) (end 103.865 102.515) (width 0.25) (layer "B.Cu") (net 1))
 (segment (start 103.865 125.375) (end 103.865 121.085) (width 0.25) (layer "B.Cu") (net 1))
 (segment (start 103.865 98.145) (end 105.49 96.52) (width 0.25) (layer "B.Cu") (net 1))
 (segment (start 160.02 125.73) (end 160.02 134.62) (width 0.25) (layer "B.Cu") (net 1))
 (segment (start 160.02 125.73) (end 160.02 118.11) (width 0.25) (layer "B.Cu") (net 1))
 (segment (start 103.945 117.755) (end 103.945 113.305) (width 0.25) (layer "B.Cu") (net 1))
 (segment (start 163.509009 114.620991) (end 163.509009 107.629009) (width 0.25) (layer "B.Cu") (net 1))
 (segment (start 129.54 151.13) (end 127.915 152.755) (width 0.25) (layer "B.Cu") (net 1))
 (segment (start 103.865 102.515) (end 103.865 98.145) (width 0.25) (layer "B.Cu") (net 1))
 (segment (start 142.771148 148.235) (end 132.435 148.235) (width 0.25) (layer "B.Cu") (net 1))
 (segment (start 114.22 80.01) (end 112.95 81.28) (width 0.25) (layer "B.Cu") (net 1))
 (segment (start 103.945 113.305) (end 105.49 111.76) (width 0.25) (layer "B.Cu") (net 1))
 (segment (start 160.02 91.44) (end 160.02 87.63) (width 0.25) (layer "B.Cu") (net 1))
 (segment (start 105.49 127) (end 103.865 125.375) (width 0.25) (layer "B.Cu") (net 1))
 (segment (start 143.365 101.455) (end 160.02 118.11) (width 0.25) (layer "B.Cu") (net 1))
 (segment (start 160.02 118.11) (end 163.509009 114.620991) (width 0.25) (layer "B.Cu") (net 1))
 (segment (start 143.51 151.13) (end 143.51 148.973852) (width 0.25) (layer "B.Cu") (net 1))
 (segment (start 142.24 93.98) (end 143.365 95.105) (width 0.25) (layer "B.Cu") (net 1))
 (segment (start 147.32 74.93) (end 125.73 74.93) (width 0.25) (layer "B.Cu") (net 1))
 (segment (start 105.49 111.76) (end 103.865 110.135) (width 0.25) (layer "B.Cu") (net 1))
 (segment (start 103.865 121.085) (end 105.57 119.38) (width 0.25) (layer "B.Cu") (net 1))
 (segment (start 125.155 75.505) (end 125.155 80.01) (width 0.25) (layer "B.Cu") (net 1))
 (segment (start 114.22 80.01) (end 125.155 80.01) (width 0.25) (layer "B.Cu") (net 1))
 (segment (start 160.02 134.62) (end 143.51 151.13) (width 0.25) (layer "B.Cu") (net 1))
 (segment (start 160.02 87.63) (end 147.32 74.93) (width 0.25) (layer "B.Cu") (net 1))
 (segment (start 103.865 105.765) (end 105.49 104.14) (width 0.25) (layer "B.Cu") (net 1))
 (segment (start 143.51 148.973852) (end 142.771148 148.235) (width 0.25) (layer "B.Cu") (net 1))
 (segment (start 143.365 95.105) (end 143.365 101.455) (width 0.25) (layer "B.Cu") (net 1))
 (segment (start 127.915 152.755) (end 126.125 152.755) (width 0.25) (layer "B.Cu") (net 1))
 (segment (start 160.02 104.14) (end 160.02 91.44) (width 0.25) (layer "B.Cu") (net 1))
 (segment (start 163.509009 107.629009) (end 160.02 104.14) (width 0.25) (layer "B.Cu") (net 1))
 (segment (start 103.865 110.135) (end 103.865 105.765) (width 0.25) (layer "B.Cu") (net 1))
 (segment (start 125.73 74.93) (end 125.155 75.505) (width 0.25) (layer "B.Cu") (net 1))
 (segment (start 106.76 110.49) (end 113.19 110.49) (width 0.25) (layer "F.Cu") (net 13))
 (segment (start 106.76 102.87) (end 113.19 102.87) (width 0.25) (layer "F.Cu") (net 12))
 (segment (start 106.76 95.25) (end 113.11 95.25) (width 0.25) (layer "F.Cu") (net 9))
 (segment (start 144.78 76.2) (end 143.96 75.38) (width 0.25) (layer "B.Cu") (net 17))
 (segment (start 144.78 77.47) (end 144.78 76.2) (width 0.25) (layer "B.Cu") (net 17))
 (segment (start 143.42 78.83) (end 144.78 77.47) (width 0.25) (layer "B.Cu") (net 17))
 (segment (start 143.42 88.81) (end 143.42 78.83) (width 0.25) (layer "B.Cu") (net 17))
 (segment (start 143.96 75.38) (end 134.17 75.38) (width 0.25) (layer "B.Cu") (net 17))
 (segment (start 155.02 104.14) (end 143.51 92.63) (width 0.25) (layer "B.Cu") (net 17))
 (segment (start 134.17 75.38) (end 132.08 77.47) (width 0.25) (layer "B.Cu") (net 17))
 (segment (start 143.51 88.9) (end 143.42 88.81) (width 0.25) (layer "B.Cu") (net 17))
 (segment (start 143.51 92.63) (end 143.51 88.9) (width 0.25) (layer "B.Cu") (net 17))
 (segment (start 128.3 82.405) (end 130.695 80.01) (width 0.25) (layer "B.Cu") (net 20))
 (segment (start 107.95 81.28) (end 109.075 82.405) (width 0.25) (layer "B.Cu") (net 20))
 (segment (start 109.075 82.405) (end 128.3 82.405) (width 0.25) (layer "B.Cu") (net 20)))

